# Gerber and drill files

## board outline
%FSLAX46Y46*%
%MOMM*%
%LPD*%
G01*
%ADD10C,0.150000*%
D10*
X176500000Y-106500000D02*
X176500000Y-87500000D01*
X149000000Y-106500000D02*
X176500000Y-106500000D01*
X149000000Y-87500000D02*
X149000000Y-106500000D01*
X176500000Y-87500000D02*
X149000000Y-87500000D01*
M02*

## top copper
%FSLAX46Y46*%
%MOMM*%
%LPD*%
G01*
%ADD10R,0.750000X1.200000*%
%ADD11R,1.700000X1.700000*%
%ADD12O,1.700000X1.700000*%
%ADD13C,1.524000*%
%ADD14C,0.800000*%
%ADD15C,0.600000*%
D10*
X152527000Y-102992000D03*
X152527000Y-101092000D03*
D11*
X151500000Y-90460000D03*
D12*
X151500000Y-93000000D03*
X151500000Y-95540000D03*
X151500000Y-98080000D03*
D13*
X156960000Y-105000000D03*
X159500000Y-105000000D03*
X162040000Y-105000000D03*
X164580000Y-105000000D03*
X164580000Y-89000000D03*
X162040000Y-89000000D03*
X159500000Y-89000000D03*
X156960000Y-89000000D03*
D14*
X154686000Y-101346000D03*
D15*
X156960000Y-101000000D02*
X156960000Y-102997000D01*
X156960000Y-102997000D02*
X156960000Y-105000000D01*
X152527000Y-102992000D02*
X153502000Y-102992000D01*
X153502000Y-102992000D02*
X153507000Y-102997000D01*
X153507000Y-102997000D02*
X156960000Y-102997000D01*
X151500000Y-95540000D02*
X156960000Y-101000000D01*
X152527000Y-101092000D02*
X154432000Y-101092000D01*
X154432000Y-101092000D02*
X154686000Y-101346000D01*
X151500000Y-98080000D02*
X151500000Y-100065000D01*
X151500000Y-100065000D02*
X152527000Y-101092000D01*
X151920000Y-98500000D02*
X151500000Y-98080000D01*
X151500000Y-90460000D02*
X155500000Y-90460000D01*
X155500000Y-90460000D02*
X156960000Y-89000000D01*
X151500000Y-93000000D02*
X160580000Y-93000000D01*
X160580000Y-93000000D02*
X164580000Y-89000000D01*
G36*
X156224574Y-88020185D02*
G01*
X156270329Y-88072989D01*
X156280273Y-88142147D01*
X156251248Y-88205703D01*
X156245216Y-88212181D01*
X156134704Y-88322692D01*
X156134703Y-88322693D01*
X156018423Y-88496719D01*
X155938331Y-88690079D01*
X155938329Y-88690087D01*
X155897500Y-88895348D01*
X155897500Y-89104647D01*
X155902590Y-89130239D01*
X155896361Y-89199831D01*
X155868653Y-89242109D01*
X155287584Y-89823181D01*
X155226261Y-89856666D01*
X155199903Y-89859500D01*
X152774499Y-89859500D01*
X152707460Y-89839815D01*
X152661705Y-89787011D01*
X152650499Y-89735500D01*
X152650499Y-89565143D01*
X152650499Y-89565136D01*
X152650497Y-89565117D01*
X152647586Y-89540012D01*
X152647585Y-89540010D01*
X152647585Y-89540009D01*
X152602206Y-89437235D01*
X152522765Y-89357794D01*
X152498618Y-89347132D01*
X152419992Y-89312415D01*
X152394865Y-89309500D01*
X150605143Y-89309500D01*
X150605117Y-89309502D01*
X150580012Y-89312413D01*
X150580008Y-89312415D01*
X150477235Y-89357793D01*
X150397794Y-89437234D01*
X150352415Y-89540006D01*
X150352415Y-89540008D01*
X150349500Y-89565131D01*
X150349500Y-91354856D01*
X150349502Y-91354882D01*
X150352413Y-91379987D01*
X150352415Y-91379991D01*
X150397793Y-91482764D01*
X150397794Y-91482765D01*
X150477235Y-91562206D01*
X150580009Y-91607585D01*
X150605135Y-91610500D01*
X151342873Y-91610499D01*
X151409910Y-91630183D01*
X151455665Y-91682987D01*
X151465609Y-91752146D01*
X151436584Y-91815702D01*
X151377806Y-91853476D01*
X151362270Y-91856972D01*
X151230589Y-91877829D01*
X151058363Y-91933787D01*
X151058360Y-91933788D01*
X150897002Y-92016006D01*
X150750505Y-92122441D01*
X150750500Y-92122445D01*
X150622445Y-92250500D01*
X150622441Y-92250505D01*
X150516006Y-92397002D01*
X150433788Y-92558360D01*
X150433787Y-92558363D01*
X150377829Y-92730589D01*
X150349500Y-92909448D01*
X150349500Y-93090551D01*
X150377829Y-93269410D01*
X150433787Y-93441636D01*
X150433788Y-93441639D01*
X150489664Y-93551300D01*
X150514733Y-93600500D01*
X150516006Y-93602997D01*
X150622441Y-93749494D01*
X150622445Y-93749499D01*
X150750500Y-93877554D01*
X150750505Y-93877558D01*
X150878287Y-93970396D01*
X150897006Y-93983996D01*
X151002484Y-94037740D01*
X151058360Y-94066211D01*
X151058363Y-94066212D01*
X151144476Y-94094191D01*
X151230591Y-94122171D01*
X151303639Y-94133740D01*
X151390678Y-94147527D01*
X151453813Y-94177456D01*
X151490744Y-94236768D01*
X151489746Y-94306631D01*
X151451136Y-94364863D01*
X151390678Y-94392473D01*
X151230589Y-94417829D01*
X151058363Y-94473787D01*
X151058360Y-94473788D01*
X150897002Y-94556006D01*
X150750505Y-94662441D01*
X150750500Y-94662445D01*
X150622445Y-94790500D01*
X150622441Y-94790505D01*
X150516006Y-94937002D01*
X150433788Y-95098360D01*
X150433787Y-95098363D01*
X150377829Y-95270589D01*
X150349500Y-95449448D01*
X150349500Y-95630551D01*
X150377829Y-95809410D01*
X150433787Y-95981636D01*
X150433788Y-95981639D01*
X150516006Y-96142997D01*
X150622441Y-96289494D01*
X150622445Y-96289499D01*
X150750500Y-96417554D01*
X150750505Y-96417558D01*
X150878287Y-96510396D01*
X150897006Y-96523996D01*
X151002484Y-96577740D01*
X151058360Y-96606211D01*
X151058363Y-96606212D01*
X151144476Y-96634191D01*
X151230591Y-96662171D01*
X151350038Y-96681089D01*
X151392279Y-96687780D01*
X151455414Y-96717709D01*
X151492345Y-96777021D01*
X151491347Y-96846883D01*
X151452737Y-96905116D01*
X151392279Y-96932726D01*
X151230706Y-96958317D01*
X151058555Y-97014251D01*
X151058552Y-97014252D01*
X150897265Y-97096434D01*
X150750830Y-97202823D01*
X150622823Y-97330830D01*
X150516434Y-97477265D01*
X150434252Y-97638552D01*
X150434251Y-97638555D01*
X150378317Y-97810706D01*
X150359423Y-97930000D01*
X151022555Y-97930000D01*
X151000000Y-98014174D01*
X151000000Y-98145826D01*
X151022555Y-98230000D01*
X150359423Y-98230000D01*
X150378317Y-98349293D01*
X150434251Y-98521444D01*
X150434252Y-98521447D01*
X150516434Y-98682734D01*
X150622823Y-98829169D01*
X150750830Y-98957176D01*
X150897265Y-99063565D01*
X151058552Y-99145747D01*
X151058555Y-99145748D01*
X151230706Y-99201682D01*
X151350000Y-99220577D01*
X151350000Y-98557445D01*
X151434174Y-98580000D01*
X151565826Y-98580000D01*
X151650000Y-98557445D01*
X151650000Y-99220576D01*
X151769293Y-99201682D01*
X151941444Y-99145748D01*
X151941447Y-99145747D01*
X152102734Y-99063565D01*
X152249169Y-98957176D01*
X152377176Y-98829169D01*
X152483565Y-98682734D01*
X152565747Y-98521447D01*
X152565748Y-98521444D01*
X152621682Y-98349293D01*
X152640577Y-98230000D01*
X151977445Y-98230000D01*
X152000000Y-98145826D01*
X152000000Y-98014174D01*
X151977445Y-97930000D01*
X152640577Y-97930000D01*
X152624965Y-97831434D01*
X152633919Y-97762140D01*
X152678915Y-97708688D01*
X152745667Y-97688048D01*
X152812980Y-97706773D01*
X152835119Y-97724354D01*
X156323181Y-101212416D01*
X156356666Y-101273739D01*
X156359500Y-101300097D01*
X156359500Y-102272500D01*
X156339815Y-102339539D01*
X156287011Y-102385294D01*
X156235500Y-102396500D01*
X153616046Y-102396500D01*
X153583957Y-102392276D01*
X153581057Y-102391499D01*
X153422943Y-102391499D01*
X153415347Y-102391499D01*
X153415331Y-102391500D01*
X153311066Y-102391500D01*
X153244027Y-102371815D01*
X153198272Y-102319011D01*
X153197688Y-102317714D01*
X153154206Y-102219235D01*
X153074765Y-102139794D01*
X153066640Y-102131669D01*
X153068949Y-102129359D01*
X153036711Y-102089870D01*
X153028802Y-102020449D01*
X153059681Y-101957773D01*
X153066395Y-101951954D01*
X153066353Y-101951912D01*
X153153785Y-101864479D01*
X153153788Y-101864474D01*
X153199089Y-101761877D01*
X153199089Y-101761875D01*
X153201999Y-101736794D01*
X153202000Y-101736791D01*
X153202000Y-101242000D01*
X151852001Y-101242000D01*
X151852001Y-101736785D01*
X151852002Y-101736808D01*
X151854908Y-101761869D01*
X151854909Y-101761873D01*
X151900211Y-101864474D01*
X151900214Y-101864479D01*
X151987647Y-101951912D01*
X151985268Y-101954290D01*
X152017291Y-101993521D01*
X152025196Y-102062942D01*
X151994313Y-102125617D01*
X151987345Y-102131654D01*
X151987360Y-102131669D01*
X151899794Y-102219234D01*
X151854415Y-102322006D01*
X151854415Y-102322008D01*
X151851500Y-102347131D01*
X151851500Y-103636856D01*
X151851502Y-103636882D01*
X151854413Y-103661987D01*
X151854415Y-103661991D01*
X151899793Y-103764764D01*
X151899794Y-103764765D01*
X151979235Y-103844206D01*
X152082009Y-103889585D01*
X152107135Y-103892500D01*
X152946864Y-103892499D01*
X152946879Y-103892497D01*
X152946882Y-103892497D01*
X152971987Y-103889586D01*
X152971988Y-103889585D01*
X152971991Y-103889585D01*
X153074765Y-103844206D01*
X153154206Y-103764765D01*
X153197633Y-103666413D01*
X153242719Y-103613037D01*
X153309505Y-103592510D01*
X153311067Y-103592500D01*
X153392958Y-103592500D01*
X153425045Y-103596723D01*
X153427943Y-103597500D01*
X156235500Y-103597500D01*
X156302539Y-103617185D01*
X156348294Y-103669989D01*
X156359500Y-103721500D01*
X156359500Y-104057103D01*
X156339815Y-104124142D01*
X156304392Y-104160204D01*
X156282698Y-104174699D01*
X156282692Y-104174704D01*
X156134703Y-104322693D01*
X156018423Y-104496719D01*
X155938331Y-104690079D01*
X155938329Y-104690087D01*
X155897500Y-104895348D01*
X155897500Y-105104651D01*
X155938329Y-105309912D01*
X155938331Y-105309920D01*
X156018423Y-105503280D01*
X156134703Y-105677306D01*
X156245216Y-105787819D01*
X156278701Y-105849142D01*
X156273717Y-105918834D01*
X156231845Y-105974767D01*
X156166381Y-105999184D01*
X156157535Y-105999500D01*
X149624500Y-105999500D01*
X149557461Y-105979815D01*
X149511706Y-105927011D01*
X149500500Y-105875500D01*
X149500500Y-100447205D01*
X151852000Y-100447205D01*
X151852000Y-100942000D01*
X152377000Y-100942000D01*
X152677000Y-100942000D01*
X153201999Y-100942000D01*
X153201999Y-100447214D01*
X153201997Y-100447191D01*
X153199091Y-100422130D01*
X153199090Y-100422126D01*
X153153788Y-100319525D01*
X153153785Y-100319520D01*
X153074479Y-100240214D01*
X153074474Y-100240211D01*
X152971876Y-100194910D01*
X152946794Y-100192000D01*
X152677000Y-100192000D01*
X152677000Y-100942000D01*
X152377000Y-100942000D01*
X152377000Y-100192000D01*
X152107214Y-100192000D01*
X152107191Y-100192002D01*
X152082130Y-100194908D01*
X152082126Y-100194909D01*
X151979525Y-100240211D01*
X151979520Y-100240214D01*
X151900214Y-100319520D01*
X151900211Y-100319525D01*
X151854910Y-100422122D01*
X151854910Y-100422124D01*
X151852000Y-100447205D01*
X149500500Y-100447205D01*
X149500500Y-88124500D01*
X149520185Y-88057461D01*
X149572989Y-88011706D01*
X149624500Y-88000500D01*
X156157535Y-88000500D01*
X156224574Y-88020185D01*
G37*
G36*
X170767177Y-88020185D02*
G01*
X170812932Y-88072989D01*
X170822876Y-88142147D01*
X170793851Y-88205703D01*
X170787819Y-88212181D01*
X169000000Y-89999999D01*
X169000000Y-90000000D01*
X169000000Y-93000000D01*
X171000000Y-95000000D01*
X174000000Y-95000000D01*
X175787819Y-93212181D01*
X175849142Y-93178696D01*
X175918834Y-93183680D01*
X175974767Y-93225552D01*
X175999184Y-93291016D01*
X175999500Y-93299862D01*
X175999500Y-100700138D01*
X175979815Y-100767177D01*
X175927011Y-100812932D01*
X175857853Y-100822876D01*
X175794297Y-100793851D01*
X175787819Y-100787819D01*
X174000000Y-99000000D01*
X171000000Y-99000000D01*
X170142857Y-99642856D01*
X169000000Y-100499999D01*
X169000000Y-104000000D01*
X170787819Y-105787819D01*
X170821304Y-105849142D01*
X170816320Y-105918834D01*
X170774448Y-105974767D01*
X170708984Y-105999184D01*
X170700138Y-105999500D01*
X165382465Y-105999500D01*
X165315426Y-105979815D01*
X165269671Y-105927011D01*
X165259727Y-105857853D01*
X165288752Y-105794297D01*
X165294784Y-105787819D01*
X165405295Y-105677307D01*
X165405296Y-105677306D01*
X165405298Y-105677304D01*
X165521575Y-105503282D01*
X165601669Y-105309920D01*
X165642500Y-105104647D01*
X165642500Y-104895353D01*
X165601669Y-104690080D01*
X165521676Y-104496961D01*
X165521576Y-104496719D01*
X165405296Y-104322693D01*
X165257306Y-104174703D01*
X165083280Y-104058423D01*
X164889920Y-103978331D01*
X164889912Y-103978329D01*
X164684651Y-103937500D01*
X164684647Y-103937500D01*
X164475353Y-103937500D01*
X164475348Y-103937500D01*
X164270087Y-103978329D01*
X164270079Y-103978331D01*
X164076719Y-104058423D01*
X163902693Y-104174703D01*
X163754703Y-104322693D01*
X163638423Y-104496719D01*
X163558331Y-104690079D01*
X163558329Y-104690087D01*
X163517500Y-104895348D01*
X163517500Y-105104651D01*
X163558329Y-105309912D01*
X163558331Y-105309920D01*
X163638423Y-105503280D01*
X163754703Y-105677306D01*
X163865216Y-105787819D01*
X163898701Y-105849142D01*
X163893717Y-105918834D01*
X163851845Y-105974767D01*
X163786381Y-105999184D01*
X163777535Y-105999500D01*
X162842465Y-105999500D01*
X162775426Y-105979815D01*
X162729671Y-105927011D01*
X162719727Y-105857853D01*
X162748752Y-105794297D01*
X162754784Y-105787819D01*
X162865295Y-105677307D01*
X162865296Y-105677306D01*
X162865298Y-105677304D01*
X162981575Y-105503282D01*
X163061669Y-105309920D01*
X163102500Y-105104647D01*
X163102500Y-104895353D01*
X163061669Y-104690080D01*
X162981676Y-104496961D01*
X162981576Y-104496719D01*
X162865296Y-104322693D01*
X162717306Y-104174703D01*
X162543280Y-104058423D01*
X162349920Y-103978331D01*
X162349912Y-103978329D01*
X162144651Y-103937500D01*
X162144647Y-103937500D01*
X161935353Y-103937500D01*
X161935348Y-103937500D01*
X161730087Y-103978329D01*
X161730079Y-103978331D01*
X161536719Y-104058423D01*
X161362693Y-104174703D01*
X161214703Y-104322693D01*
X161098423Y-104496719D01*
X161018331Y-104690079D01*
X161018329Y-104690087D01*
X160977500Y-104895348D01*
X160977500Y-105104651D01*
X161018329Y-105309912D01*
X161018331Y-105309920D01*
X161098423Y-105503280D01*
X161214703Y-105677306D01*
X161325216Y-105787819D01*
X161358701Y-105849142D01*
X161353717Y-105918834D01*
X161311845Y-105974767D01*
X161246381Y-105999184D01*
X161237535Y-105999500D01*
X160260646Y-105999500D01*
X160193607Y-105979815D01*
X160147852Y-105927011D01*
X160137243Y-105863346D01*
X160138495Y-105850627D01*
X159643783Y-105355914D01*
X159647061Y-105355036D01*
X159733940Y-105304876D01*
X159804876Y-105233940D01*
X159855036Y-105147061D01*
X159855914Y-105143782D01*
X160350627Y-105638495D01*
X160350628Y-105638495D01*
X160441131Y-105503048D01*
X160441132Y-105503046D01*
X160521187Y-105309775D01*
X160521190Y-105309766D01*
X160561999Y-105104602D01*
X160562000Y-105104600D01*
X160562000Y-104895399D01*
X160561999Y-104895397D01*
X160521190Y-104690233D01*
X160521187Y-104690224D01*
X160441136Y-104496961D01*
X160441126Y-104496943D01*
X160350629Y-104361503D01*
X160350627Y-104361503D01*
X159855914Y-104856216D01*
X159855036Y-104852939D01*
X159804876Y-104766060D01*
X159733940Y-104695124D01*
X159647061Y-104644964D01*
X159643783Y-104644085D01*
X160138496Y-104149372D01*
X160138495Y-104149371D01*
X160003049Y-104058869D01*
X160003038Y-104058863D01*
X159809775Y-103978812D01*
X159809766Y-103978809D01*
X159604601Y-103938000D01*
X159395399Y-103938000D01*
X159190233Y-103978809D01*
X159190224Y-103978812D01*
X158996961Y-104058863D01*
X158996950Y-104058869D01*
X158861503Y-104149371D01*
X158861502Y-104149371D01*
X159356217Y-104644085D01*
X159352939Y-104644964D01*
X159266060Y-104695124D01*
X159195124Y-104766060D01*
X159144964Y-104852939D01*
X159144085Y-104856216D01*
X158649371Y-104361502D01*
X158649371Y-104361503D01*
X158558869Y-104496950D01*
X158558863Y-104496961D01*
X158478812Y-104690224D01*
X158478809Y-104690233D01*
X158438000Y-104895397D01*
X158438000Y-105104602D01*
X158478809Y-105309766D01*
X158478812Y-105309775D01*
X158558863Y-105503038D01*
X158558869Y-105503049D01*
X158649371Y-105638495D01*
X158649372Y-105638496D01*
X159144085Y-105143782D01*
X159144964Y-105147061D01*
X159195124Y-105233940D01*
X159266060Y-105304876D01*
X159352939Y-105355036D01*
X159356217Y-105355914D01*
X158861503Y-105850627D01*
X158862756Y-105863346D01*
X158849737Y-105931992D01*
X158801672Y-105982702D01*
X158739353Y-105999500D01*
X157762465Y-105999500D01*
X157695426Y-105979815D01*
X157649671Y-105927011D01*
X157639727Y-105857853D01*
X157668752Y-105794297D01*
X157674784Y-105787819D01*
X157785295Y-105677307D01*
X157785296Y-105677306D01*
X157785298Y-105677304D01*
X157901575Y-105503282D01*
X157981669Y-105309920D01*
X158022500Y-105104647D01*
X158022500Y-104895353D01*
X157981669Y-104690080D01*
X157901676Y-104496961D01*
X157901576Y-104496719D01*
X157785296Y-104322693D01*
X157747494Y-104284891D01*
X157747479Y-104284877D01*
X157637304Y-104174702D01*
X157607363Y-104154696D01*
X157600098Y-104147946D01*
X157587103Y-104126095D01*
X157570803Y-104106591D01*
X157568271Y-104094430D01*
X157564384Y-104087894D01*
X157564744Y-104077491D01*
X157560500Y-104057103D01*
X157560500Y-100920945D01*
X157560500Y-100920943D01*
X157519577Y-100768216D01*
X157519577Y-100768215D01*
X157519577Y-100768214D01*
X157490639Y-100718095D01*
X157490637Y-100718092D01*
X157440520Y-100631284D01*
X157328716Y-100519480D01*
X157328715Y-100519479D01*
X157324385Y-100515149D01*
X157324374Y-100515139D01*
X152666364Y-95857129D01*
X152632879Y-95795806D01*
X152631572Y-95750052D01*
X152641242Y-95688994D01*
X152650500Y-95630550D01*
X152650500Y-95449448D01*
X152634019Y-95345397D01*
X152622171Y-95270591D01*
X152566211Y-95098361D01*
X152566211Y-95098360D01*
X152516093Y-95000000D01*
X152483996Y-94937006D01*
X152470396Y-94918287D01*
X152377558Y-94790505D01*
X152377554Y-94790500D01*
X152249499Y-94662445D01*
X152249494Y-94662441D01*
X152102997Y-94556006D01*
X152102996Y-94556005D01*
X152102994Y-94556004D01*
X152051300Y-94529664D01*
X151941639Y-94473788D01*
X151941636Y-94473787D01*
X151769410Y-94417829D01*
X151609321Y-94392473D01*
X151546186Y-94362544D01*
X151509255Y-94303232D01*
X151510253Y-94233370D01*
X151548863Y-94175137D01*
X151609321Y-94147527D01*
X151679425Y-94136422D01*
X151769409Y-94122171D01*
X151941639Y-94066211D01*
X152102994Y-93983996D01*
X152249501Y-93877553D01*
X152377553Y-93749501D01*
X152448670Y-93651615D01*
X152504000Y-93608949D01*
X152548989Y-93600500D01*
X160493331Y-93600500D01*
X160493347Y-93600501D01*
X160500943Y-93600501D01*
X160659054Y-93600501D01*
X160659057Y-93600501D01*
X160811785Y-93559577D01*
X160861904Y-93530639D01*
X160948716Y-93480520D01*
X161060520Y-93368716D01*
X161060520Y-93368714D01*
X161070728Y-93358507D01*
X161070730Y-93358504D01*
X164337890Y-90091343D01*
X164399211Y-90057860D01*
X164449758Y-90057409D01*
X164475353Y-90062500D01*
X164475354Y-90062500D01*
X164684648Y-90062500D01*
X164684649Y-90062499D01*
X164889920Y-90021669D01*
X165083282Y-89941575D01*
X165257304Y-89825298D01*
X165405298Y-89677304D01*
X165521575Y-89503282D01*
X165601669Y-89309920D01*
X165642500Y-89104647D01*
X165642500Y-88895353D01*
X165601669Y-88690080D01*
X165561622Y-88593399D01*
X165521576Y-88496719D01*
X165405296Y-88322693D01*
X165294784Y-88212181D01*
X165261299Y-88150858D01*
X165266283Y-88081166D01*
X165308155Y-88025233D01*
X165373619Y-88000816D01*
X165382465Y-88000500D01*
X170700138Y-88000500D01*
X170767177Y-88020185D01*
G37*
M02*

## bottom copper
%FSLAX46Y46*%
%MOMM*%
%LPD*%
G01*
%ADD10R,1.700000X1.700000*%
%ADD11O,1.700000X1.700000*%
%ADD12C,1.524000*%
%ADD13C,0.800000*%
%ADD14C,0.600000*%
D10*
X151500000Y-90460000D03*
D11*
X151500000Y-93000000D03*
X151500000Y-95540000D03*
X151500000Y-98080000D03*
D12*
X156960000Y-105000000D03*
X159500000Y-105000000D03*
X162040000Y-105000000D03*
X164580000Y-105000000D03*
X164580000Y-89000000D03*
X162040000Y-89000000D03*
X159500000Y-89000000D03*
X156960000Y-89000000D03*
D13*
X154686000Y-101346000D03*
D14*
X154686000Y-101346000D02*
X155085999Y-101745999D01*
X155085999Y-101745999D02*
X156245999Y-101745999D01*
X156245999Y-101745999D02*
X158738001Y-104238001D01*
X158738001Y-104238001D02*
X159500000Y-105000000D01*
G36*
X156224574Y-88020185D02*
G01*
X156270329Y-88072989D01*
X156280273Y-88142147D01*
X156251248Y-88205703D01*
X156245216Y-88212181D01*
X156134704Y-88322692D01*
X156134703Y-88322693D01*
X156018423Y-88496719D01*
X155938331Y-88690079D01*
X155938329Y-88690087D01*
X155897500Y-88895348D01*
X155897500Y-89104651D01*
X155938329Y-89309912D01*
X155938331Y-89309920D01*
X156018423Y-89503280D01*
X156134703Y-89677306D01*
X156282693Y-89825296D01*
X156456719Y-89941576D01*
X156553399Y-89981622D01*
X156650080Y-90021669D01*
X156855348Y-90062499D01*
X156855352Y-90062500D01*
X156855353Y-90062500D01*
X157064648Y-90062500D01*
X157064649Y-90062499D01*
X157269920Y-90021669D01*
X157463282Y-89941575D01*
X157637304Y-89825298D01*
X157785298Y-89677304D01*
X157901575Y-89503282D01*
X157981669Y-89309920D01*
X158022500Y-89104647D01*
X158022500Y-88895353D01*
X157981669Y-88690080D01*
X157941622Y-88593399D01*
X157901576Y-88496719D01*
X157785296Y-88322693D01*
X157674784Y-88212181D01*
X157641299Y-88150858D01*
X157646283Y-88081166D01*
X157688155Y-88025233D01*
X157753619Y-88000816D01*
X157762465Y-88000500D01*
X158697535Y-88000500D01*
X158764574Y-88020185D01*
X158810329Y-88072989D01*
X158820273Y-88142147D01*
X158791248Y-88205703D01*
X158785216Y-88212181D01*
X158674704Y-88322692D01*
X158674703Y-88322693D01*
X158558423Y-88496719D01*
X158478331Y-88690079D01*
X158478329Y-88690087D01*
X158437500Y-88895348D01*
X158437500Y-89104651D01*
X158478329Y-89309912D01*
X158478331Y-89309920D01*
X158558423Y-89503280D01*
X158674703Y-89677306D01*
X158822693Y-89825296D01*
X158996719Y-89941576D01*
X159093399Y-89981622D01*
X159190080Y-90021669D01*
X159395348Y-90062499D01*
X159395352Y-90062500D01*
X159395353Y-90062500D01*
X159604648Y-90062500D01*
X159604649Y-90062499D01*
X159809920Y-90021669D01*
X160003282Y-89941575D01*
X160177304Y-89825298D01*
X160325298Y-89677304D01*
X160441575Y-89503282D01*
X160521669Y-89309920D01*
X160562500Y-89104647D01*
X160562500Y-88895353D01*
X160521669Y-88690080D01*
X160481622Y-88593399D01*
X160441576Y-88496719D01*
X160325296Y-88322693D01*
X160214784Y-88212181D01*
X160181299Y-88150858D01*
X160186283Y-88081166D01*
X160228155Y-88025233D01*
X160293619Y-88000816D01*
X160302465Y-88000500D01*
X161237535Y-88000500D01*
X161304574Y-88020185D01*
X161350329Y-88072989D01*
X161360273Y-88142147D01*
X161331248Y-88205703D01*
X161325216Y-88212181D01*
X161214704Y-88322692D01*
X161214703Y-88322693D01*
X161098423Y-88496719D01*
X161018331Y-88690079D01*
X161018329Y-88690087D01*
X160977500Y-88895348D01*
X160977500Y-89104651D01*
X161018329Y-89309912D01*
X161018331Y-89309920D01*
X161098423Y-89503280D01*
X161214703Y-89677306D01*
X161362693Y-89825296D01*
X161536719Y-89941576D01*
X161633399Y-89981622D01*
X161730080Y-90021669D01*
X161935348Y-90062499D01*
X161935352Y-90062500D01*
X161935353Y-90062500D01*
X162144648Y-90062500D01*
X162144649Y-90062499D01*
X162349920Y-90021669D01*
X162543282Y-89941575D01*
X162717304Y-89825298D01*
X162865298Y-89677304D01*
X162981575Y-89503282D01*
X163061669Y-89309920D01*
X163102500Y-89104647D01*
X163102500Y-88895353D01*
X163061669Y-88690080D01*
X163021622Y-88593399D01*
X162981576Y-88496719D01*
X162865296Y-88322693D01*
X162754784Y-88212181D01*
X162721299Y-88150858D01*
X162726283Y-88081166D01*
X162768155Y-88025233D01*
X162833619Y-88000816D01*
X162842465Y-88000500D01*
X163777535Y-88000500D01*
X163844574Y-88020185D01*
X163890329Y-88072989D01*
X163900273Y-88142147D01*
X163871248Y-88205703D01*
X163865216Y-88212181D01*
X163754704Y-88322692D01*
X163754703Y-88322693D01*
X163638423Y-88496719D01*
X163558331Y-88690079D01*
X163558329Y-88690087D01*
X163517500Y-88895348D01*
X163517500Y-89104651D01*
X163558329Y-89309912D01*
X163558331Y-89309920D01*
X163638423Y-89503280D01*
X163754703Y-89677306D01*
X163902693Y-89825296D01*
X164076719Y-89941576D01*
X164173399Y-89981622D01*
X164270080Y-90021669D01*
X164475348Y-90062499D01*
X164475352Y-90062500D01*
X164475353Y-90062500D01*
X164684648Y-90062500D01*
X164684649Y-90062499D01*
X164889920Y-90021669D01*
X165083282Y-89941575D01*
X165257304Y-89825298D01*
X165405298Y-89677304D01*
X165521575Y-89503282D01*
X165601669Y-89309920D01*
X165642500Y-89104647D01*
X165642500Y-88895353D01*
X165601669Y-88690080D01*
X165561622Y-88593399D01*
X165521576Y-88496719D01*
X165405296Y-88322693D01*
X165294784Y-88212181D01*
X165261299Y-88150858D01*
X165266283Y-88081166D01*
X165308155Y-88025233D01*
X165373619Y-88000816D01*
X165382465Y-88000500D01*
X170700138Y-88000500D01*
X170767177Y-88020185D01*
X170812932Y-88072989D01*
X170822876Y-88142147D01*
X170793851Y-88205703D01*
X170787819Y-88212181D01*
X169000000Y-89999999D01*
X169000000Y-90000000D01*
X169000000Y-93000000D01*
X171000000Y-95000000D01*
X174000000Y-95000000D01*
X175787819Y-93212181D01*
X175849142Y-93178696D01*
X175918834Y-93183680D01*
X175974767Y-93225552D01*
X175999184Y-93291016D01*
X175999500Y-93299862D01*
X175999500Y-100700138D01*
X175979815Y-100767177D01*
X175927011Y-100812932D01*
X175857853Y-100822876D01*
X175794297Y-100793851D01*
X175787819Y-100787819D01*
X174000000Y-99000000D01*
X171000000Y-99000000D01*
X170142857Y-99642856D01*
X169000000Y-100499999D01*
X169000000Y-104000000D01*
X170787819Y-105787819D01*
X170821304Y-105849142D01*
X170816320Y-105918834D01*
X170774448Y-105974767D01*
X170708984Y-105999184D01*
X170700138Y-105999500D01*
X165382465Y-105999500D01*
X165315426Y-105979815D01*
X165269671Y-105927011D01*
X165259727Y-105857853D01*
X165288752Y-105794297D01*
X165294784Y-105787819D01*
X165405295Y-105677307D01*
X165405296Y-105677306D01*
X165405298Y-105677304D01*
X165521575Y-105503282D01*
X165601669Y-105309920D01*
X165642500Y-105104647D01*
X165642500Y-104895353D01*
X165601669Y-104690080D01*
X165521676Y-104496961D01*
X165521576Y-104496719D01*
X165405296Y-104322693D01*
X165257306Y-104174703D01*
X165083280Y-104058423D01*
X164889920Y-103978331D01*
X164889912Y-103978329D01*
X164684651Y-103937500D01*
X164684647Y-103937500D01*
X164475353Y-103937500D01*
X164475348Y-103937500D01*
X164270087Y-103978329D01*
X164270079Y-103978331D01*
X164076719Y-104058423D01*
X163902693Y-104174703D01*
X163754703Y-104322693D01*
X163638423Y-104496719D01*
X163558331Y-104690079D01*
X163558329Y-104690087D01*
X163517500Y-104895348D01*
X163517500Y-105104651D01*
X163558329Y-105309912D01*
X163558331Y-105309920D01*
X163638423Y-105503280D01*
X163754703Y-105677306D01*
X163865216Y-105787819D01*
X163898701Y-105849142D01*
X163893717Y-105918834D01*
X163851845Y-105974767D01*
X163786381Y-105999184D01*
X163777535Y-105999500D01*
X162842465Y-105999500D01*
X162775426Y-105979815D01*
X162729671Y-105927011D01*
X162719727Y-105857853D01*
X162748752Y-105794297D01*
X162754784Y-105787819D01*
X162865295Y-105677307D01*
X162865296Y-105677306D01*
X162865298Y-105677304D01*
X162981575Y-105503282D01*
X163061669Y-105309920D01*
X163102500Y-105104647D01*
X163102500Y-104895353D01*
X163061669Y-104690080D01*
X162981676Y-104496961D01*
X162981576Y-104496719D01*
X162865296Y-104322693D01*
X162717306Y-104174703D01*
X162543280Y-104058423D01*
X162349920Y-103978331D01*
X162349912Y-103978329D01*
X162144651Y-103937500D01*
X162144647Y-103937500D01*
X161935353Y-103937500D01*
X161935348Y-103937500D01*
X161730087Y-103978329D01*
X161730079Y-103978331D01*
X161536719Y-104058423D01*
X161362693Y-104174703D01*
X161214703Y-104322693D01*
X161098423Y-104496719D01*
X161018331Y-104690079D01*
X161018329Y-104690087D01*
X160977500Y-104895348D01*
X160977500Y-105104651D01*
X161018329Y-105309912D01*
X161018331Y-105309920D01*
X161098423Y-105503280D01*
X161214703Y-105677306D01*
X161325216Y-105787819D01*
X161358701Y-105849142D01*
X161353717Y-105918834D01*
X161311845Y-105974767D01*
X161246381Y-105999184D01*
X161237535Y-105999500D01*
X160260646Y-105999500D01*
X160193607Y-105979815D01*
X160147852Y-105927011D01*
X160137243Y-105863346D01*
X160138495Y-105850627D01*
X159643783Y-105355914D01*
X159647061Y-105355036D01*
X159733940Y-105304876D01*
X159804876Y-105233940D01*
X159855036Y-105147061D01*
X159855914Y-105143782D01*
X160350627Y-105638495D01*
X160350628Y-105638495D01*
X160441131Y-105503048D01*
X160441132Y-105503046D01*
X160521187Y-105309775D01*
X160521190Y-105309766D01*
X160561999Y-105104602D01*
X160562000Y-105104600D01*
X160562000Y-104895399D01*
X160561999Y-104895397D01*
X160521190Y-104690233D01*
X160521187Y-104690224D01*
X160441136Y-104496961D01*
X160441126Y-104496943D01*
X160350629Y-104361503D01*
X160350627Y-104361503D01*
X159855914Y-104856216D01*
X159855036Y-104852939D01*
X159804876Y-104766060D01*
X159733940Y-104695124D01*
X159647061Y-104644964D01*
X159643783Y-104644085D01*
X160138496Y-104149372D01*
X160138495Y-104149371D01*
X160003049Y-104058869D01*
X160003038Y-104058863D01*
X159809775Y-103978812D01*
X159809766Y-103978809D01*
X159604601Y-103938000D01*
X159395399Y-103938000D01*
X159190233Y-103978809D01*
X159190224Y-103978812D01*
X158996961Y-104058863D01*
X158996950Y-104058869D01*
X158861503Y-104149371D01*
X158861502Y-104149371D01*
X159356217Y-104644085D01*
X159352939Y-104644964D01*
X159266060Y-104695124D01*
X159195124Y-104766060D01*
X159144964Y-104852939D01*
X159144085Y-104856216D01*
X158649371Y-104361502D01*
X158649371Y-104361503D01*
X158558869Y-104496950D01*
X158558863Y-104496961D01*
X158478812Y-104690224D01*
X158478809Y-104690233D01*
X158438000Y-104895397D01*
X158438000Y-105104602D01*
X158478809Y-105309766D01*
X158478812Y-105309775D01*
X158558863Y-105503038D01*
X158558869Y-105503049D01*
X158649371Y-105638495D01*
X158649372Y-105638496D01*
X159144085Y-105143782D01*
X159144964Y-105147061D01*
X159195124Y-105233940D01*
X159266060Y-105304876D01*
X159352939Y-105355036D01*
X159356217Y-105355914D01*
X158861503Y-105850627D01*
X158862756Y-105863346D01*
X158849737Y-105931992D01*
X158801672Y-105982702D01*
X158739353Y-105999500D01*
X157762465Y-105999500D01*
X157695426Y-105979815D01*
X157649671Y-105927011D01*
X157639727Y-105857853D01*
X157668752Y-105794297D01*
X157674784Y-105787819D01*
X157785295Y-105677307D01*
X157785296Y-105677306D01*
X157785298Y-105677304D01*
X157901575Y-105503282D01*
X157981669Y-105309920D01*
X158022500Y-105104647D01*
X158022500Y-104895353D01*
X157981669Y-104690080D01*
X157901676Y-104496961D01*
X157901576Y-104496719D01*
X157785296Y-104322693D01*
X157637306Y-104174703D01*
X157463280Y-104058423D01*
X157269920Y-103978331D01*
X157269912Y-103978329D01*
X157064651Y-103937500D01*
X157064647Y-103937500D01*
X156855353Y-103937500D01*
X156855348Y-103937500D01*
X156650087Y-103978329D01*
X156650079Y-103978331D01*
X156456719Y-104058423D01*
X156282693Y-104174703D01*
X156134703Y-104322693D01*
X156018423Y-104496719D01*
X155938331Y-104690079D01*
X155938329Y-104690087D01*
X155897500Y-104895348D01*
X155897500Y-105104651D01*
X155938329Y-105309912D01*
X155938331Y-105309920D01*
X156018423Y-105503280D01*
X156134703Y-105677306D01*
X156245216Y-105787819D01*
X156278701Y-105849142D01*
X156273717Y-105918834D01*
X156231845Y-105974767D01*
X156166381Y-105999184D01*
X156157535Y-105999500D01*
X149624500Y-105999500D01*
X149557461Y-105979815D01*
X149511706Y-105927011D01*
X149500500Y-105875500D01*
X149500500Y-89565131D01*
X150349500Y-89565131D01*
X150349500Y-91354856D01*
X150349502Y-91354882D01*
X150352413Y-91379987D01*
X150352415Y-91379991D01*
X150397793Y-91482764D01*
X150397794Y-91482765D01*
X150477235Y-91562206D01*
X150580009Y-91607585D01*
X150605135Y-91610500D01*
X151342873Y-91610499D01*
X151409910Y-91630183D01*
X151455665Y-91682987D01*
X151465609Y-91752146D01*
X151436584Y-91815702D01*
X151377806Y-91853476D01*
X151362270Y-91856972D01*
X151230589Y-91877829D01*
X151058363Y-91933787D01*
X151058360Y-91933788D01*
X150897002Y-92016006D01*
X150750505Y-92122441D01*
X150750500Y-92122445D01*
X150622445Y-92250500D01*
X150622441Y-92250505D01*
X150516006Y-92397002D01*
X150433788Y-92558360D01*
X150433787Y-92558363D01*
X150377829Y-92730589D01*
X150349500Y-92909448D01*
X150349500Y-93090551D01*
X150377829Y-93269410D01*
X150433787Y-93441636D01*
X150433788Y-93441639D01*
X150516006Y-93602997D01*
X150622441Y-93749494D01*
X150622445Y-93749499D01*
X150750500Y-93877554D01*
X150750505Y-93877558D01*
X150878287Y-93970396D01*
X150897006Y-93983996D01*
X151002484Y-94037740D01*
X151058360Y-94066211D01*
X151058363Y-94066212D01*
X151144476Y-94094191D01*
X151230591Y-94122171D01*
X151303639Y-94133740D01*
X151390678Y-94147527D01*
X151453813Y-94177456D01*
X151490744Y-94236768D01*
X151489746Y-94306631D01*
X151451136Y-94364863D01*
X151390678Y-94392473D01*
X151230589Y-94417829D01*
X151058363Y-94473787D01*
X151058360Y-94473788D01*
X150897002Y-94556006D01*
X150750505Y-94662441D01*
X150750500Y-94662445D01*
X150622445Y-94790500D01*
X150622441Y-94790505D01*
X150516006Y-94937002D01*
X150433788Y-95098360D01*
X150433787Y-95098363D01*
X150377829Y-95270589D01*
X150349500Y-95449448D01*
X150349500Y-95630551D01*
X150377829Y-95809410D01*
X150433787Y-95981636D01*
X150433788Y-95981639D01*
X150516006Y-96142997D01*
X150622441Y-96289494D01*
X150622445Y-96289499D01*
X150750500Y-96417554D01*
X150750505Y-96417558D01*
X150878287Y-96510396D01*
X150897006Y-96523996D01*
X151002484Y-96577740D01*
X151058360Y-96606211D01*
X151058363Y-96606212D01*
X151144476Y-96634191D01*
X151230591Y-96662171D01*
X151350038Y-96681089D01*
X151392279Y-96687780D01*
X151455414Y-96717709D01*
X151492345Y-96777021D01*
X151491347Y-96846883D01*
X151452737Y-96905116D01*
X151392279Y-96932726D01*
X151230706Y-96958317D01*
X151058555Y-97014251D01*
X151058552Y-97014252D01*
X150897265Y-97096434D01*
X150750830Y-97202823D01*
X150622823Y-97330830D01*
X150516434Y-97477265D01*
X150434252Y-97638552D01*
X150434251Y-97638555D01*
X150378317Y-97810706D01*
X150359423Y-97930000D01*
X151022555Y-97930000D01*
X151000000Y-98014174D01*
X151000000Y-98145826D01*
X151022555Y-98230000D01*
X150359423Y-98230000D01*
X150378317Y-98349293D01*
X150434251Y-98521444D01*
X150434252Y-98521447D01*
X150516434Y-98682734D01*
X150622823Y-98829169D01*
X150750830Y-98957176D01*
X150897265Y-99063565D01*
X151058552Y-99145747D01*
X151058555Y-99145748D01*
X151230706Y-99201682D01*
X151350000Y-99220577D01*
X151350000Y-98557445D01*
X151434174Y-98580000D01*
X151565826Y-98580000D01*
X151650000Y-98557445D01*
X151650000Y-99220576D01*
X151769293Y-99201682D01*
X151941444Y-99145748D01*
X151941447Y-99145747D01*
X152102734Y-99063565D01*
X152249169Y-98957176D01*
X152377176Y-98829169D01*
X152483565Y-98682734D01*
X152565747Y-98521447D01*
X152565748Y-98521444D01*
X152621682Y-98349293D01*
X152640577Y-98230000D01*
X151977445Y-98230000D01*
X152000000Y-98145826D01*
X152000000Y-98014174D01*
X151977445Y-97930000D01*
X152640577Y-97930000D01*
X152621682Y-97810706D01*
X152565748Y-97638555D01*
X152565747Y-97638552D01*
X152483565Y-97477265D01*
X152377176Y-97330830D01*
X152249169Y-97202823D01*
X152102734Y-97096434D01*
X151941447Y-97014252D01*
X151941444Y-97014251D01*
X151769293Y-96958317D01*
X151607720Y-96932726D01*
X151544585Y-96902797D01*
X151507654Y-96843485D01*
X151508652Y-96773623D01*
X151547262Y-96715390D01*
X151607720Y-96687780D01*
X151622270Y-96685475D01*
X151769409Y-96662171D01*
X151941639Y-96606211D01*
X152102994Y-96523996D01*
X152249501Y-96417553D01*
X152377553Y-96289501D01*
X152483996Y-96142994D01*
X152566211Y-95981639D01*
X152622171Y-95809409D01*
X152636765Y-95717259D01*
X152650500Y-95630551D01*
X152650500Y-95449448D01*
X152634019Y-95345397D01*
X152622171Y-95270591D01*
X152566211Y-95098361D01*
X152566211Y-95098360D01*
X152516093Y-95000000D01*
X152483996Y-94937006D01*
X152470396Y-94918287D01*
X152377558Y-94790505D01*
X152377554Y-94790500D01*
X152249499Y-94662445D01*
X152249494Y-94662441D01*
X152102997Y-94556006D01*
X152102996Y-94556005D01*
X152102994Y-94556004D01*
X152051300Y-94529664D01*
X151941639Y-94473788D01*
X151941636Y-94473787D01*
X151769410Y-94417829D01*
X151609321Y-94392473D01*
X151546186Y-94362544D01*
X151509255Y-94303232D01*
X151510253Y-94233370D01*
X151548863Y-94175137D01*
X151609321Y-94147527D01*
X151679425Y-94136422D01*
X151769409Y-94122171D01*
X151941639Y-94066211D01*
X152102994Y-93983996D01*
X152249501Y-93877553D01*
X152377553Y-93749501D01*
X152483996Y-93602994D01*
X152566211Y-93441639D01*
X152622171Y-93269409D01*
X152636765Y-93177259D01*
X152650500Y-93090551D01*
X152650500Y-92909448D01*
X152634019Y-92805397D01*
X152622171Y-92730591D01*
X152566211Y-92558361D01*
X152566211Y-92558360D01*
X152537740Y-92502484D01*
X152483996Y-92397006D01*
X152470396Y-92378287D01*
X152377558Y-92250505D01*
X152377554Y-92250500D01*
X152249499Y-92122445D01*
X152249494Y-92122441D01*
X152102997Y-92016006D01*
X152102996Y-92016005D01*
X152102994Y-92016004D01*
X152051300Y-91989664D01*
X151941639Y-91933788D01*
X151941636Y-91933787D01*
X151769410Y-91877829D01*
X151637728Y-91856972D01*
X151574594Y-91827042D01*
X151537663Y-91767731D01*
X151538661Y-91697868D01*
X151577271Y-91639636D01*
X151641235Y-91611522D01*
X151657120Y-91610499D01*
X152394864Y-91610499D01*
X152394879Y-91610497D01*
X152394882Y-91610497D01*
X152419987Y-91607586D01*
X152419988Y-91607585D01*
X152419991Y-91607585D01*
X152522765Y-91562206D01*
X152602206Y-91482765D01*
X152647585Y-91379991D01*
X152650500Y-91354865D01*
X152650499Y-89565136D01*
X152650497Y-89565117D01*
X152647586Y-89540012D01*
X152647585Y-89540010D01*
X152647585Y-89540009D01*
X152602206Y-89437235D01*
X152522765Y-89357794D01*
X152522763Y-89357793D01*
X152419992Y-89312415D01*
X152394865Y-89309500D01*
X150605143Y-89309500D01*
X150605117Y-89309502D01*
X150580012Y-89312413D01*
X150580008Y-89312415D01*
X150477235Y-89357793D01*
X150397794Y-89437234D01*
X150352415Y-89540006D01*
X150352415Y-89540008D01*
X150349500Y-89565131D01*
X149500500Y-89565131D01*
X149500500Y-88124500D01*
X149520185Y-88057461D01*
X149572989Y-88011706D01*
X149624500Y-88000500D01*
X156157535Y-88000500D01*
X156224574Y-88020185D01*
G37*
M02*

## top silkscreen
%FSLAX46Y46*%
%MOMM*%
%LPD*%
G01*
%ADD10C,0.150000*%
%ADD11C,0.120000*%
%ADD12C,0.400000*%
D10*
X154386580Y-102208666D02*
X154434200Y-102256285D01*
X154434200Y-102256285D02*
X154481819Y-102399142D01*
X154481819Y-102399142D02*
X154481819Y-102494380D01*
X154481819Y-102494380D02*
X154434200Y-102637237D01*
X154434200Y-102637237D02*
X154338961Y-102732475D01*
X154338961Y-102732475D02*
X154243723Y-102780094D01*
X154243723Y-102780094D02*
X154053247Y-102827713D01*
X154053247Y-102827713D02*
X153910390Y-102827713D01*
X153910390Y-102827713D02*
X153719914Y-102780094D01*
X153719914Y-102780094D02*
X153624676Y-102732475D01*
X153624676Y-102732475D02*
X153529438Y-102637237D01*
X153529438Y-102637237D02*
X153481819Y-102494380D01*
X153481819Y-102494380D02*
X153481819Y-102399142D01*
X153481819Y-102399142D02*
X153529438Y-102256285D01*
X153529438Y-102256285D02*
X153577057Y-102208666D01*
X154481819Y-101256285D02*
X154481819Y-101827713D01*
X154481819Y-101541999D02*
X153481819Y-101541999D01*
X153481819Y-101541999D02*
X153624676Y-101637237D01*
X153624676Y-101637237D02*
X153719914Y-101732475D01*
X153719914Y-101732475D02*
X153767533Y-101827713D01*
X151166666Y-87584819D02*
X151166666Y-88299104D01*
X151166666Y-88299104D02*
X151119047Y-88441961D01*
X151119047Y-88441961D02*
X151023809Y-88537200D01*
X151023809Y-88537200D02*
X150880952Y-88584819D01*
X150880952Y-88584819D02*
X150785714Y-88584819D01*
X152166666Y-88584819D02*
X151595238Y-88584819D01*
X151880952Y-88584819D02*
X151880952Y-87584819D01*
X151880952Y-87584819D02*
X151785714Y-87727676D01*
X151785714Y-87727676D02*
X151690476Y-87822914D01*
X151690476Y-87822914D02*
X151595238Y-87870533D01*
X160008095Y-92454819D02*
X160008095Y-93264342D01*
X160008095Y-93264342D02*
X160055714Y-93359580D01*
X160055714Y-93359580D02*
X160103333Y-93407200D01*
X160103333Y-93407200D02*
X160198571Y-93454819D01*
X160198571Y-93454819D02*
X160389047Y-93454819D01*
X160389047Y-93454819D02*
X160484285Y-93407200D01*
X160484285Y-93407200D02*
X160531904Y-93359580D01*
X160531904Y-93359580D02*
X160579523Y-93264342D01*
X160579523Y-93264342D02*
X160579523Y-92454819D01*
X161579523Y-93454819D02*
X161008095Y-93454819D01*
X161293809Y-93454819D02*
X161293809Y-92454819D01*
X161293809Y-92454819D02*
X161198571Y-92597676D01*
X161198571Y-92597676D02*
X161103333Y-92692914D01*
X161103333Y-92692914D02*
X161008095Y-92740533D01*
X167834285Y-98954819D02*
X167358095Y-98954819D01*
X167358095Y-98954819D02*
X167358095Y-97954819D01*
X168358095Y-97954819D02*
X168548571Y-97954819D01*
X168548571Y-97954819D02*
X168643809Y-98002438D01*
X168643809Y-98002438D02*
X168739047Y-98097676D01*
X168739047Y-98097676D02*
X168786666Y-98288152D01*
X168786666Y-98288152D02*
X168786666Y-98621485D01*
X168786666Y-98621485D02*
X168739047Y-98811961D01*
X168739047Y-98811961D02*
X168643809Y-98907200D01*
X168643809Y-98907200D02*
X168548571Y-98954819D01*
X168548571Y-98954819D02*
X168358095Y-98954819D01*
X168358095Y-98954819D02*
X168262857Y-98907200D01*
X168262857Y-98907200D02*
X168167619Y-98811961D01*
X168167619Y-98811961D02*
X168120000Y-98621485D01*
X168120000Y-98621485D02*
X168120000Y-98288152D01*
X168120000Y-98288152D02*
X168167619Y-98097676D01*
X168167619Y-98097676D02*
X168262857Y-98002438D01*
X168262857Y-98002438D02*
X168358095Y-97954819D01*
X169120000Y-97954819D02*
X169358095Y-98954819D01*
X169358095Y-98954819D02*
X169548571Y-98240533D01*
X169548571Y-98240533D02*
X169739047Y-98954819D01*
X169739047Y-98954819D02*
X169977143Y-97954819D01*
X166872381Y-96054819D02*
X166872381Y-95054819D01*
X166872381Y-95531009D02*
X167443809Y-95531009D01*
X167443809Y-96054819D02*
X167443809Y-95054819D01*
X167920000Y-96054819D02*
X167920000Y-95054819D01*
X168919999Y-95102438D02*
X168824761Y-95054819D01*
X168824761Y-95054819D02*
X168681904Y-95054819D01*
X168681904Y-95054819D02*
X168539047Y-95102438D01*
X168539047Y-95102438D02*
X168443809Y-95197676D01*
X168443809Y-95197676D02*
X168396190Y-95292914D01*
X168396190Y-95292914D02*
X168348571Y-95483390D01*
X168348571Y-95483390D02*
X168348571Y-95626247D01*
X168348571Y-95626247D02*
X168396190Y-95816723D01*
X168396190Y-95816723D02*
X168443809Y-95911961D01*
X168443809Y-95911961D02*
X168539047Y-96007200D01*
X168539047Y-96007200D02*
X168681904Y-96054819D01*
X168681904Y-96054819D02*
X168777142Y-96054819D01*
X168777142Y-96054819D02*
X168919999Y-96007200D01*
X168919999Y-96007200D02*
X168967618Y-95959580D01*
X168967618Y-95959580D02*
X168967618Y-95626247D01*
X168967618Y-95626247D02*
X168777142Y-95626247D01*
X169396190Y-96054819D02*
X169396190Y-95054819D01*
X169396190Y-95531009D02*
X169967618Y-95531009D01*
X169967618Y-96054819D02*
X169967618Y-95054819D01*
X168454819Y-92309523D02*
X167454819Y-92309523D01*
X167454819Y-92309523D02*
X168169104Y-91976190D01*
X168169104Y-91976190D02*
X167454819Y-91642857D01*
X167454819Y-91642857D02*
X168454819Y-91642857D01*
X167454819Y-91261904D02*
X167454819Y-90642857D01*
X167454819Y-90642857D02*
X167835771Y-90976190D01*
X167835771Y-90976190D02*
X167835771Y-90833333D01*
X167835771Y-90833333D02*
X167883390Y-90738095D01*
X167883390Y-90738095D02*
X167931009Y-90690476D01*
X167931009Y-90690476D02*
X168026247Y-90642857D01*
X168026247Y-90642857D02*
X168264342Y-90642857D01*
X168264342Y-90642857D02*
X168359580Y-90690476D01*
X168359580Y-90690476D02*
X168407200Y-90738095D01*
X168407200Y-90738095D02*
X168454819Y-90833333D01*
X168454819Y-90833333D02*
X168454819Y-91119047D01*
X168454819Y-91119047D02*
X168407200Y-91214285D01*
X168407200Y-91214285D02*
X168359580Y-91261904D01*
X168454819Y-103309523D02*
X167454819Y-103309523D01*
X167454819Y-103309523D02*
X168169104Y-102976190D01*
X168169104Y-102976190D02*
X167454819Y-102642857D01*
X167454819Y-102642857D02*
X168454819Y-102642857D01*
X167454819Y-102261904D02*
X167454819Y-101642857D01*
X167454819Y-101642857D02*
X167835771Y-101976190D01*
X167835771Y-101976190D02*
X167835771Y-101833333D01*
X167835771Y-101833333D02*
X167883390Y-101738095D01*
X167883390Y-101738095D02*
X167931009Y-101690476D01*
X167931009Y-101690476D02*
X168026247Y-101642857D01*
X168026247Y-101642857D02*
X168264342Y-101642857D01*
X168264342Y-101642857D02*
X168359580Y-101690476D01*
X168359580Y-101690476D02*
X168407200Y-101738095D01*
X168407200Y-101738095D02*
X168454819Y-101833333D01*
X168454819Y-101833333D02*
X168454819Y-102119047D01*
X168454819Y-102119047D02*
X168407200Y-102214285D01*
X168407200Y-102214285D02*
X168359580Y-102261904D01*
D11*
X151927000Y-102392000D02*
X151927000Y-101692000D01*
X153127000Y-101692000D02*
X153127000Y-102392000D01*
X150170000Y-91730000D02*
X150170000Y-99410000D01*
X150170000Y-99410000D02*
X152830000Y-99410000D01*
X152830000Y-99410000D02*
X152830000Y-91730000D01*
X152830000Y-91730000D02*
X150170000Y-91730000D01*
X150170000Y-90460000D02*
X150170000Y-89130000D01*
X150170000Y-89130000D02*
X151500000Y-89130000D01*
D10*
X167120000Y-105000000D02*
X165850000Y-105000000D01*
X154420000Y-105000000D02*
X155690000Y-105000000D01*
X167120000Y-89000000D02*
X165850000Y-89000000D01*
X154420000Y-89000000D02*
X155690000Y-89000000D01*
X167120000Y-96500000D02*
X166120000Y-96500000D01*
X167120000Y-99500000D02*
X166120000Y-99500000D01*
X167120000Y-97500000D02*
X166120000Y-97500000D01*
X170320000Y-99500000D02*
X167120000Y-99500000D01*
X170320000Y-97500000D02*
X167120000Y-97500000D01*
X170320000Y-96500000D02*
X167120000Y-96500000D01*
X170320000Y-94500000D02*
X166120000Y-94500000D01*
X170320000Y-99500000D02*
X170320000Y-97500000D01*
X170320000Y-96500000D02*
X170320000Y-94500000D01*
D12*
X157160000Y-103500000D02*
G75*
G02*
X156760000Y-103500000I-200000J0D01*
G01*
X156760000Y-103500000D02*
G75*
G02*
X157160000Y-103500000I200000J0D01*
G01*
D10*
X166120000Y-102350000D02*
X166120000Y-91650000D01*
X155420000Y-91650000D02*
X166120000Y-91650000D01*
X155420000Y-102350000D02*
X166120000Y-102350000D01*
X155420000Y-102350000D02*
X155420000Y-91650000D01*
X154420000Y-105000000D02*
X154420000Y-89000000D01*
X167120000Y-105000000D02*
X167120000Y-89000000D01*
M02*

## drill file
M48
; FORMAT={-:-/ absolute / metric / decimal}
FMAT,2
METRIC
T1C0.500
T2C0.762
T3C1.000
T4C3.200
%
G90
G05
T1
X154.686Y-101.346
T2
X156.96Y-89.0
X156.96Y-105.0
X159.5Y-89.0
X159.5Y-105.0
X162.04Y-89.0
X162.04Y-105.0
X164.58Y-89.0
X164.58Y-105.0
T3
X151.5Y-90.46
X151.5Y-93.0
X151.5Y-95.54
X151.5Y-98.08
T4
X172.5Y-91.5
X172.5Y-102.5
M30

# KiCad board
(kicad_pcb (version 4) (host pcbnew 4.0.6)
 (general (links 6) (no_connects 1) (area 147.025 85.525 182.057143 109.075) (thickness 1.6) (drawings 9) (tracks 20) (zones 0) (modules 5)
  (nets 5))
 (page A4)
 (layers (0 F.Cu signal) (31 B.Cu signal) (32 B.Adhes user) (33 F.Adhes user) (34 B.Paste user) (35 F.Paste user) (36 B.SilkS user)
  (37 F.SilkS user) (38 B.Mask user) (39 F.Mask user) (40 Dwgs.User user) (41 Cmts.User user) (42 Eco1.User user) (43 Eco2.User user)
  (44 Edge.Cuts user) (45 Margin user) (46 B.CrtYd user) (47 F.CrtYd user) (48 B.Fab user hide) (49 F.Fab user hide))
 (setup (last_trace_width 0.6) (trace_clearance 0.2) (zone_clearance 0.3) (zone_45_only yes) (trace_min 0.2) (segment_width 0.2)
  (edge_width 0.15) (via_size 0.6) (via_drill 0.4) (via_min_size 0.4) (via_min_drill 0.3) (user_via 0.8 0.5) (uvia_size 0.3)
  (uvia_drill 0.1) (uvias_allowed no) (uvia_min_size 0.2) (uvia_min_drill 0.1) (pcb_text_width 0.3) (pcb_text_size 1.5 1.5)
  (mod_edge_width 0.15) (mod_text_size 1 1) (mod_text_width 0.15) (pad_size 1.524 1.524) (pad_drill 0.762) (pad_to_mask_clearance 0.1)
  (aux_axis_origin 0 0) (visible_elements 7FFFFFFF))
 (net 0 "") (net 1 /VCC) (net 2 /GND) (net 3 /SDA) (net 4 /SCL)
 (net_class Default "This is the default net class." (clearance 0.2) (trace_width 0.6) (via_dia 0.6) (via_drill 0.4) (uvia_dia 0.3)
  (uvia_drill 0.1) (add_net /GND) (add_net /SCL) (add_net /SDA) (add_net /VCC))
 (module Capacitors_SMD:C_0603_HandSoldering (layer F.Cu) (at 152.527 102.042 90)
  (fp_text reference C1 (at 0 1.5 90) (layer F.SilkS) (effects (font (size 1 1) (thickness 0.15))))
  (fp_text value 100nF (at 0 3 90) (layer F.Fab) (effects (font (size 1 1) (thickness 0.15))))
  (fp_line (start -0.35 -0.6) (end 0.35 -0.6) (layer F.SilkS) (width 0.12))
  (fp_line (start 0.35 0.6) (end -0.35 0.6) (layer F.SilkS) (width 0.12))
  (pad 1 smd rect (at -0.95 0 90) (size 1.2 0.75) (layers F.Cu F.Paste F.Mask) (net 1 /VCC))
  (pad 2 smd rect (at 0.95 0 90) (size 1.2 0.75) (layers F.Cu F.Paste F.Mask) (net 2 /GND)))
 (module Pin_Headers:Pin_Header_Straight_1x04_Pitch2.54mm (layer F.Cu) (at 151.5 90.46)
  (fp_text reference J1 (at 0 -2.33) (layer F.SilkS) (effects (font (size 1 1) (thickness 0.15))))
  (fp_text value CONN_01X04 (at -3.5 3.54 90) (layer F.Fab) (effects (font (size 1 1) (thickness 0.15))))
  (fp_line (start -1.33 1.27) (end -1.33 8.95) (layer F.SilkS) (width 0.12))
  (fp_line (start -1.33 8.95) (end 1.33 8.95) (layer F.SilkS) (width 0.12))
  (fp_line (start 1.33 8.95) (end 1.33 1.27) (layer F.SilkS) (width 0.12))
  (fp_line (start 1.33 1.27) (end -1.33 1.27) (layer F.SilkS) (width 0.12))
  (fp_line (start -1.33 0) (end -1.33 -1.33) (layer F.SilkS) (width 0.12))
  (fp_line (start -1.33 -1.33) (end 0 -1.33) (layer F.SilkS) (width 0.12))
  (pad 1 thru_hole rect (at 0 0) (size 1.7 1.7) (drill 1) (layers *.Cu *.Mask) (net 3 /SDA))
  (pad 2 thru_hole oval (at 0 2.54) (size 1.7 1.7) (drill 1) (layers *.Cu *.Mask) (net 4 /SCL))
  (pad 3 thru_hole oval (at 0 5.08) (size 1.7 1.7) (drill 1) (layers *.Cu *.Mask) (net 1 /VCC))
  (pad 4 thru_hole oval (at 0 7.62) (size 1.7 1.7) (drill 1) (layers *.Cu *.Mask) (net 2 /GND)))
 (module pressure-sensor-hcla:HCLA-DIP (layer F.Cu) (at 154.42 105)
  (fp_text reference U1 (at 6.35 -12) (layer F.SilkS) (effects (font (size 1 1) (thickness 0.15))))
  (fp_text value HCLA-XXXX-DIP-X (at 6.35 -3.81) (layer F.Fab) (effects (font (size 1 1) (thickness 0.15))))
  (fp_line (start 12.7 0) (end 11.43 0) (layer F.SilkS) (width 0.15))
  (fp_line (start 0 0) (end 1.27 0) (layer F.SilkS) (width 0.15))
  (fp_line (start 12.7 -16) (end 11.43 -16) (layer F.SilkS) (width 0.15))
  (fp_line (start 0 -16) (end 1.27 -16) (layer F.SilkS) (width 0.15))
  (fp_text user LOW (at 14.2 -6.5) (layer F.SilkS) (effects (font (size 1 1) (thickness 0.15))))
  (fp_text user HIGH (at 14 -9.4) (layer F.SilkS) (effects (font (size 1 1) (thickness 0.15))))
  (fp_line (start 12.7 -8.5) (end 11.7 -8.5) (layer F.SilkS) (width 0.15))
  (fp_line (start 12.7 -5.5) (end 11.7 -5.5) (layer F.SilkS) (width 0.15))
  (fp_line (start 12.7 -7.5) (end 11.7 -7.5) (layer F.SilkS) (width 0.15))
  (fp_line (start 15.9 -5.5) (end 12.7 -5.5) (layer F.SilkS) (width 0.15))
  (fp_line (start 15.9 -7.5) (end 12.7 -7.5) (layer F.SilkS) (width 0.15))
  (fp_line (start 15.9 -8.5) (end 12.7 -8.5) (layer F.SilkS) (width 0.15))
  (fp_line (start 15.9 -10.5) (end 11.7 -10.5) (layer F.SilkS) (width 0.15))
  (fp_line (start 15.9 -5.5) (end 15.9 -7.5) (layer F.SilkS) (width 0.15))
  (fp_line (start 15.9 -8.5) (end 15.9 -10.5) (layer F.SilkS) (width 0.15))
  (fp_circle (center 2.54 -1.5) (end 2.54 -1.7) (layer F.SilkS) (width 0.4))
  (fp_line (start 11.7 -2.65) (end 11.7 -13.35) (layer F.SilkS) (width 0.15))
  (fp_line (start 1 -13.35) (end 11.7 -13.35) (layer F.SilkS) (width 0.15))
  (fp_line (start 1 -2.65) (end 11.7 -2.65) (layer F.SilkS) (width 0.15))
  (fp_line (start 1 -2.65) (end 1 -13.35) (layer F.SilkS) (width 0.15))
  (fp_line (start 0 0) (end 0 -16) (layer F.SilkS) (width 0.15))
  (fp_line (start 12.7 0) (end 12.7 -16) (layer F.SilkS) (width 0.15))
  (pad 1 thru_hole circle (at 2.54 0) (size 1.524 1.524) (drill 0.762) (layers *.Cu *.Mask) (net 1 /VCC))
  (pad 2 thru_hole circle (at 5.08 0) (size 1.524 1.524) (drill 0.762) (layers *.Cu *.Mask) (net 2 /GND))
  (pad 3 thru_hole circle (at 7.62 0) (size 1.524 1.524) (drill 0.762) (layers *.Cu *.Mask))
  (pad 4 thru_hole circle (at 10.16 0) (size 1.524 1.524) (drill 0.762) (layers *.Cu *.Mask))
  (pad 5 thru_hole circle (at 10.16 -16) (size 1.524 1.524) (drill 0.762) (layers *.Cu *.Mask) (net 4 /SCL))
  (pad 6 thru_hole circle (at 7.62 -16) (size 1.524 1.524) (drill 0.762) (layers *.Cu *.Mask))
  (pad 7 thru_hole circle (at 5.08 -16) (size 1.524 1.524) (drill 0.762) (layers *.Cu *.Mask))
  (pad 8 thru_hole circle (at 2.54 -16) (size 1.524 1.524) (drill 0.762) (layers *.Cu *.Mask) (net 3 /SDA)))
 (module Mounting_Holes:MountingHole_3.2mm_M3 (layer F.Cu) (at 172.5 91.5)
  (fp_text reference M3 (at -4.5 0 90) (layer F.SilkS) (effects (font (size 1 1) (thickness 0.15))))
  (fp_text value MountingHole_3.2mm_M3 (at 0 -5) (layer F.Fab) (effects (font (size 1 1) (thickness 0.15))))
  (pad 1 np_thru_hole circle (at 0 0) (size 3.2 3.2) (drill 3.2) (layers *.Cu *.Mask)))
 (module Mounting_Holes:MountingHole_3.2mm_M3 (layer F.Cu) (at 172.5 102.5)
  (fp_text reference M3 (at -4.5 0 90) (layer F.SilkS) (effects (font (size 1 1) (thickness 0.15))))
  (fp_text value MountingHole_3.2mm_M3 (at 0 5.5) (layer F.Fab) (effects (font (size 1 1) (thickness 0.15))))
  (pad 1 np_thru_hole circle (at 0 0) (size 3.2 3.2) (drill 3.2) (layers *.Cu *.Mask)))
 (gr_line (start 176.5 106.5) (end 176.5 87.5) (layer Edge.Cuts) (width 0.15))
 (gr_line (start 149 106.5) (end 176.5 106.5) (layer Edge.Cuts) (width 0.15))
 (gr_line (start 149 87.5) (end 149 106.5) (layer Edge.Cuts) (width 0.15))
 (gr_line (start 176.5 87.5) (end 149 87.5) (layer Edge.Cuts) (width 0.15))
 (segment (start 156.96 101) (end 156.96 102.997) (width 0.6) (layer F.Cu) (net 1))
 (segment (start 156.96 102.997) (end 156.96 105) (width 0.6) (layer F.Cu) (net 1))
 (segment (start 152.527 102.992) (end 153.502 102.992) (width 0.6) (layer F.Cu) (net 1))
 (segment (start 153.502 102.992) (end 153.507 102.997) (width 0.6) (layer F.Cu) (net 1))
 (segment (start 153.507 102.997) (end 156.96 102.997) (width 0.6) (layer F.Cu) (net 1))
 (segment (start 151.5 95.54) (end 156.96 101) (width 0.6) (layer F.Cu) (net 1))
 (segment (start 154.686 101.346) (end 155.085999 101.745999) (width 0.6) (layer B.Cu) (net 2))
 (segment (start 155.085999 101.745999) (end 156.245999 101.745999) (width 0.6) (layer B.Cu) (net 2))
 (segment (start 156.245999 101.745999) (end 158.738001 104.238001) (width 0.6) (layer B.Cu) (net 2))
 (segment (start 158.738001 104.238001) (end 159.5 105) (width 0.6) (layer B.Cu) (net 2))
 (segment (start 152.527 101.092) (end 154.432 101.092) (width 0.6) (layer F.Cu) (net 2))
 (segment (start 154.432 101.092) (end 154.686 101.346) (width 0.6) (layer F.Cu) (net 2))
 (via (at 154.686 101.346) (size 0.8) (drill 0.5) (layers F.Cu B.Cu) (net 2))
 (segment (start 151.5 98.08) (end 151.5 100.065) (width 0.6) (layer F.Cu) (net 2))
 (segment (start 151.5 100.065) (end 152.527 101.092) (width 0.6) (layer F.Cu) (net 2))
 (segment (start 151.92 98.5) (end 151.5 98.08) (width 0.6) (layer F.Cu) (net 2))
 (segment (start 151.5 90.46) (end 155.5 90.46) (width 0.6) (layer F.Cu) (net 3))
 (segment (start 155.5 90.46) (end 156.96 89) (width 0.6) (layer F.Cu) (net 3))
 (segment (start 151.5 93) (end 160.58 93) (width 0.6) (layer F.Cu) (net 4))
 (segment (start 160.58 93) (end 164.58 89) (width 0.6) (layer F.Cu) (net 4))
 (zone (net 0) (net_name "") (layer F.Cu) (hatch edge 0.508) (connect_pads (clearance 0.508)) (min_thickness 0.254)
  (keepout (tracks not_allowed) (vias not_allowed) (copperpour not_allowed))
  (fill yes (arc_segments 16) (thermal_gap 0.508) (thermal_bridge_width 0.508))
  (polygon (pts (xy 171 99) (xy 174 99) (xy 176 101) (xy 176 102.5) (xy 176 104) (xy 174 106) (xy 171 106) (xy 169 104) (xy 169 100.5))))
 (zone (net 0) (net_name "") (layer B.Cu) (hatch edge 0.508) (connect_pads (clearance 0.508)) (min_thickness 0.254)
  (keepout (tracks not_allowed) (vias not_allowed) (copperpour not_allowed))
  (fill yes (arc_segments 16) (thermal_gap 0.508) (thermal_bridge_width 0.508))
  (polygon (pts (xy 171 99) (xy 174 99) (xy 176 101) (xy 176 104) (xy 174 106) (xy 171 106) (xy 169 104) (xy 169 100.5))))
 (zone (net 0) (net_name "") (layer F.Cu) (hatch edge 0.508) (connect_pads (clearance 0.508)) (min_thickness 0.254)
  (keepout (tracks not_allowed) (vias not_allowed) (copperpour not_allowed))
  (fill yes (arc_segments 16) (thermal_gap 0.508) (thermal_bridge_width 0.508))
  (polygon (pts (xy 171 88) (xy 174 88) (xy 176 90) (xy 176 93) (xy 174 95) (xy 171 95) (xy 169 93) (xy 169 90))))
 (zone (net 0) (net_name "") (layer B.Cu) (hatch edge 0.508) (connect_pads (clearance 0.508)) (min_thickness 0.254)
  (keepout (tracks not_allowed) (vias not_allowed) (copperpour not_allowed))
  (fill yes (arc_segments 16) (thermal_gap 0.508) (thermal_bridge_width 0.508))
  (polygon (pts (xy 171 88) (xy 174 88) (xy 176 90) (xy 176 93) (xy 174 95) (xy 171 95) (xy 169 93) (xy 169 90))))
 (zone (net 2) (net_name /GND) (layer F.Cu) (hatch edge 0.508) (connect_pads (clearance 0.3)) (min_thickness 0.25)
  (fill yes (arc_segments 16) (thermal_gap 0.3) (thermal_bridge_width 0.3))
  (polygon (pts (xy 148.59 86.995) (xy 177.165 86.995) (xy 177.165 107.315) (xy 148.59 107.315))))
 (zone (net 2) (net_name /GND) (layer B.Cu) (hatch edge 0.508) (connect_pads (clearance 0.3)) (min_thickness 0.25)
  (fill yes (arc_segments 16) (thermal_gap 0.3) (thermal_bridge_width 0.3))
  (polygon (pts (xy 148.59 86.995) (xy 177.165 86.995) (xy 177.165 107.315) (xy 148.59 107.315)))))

